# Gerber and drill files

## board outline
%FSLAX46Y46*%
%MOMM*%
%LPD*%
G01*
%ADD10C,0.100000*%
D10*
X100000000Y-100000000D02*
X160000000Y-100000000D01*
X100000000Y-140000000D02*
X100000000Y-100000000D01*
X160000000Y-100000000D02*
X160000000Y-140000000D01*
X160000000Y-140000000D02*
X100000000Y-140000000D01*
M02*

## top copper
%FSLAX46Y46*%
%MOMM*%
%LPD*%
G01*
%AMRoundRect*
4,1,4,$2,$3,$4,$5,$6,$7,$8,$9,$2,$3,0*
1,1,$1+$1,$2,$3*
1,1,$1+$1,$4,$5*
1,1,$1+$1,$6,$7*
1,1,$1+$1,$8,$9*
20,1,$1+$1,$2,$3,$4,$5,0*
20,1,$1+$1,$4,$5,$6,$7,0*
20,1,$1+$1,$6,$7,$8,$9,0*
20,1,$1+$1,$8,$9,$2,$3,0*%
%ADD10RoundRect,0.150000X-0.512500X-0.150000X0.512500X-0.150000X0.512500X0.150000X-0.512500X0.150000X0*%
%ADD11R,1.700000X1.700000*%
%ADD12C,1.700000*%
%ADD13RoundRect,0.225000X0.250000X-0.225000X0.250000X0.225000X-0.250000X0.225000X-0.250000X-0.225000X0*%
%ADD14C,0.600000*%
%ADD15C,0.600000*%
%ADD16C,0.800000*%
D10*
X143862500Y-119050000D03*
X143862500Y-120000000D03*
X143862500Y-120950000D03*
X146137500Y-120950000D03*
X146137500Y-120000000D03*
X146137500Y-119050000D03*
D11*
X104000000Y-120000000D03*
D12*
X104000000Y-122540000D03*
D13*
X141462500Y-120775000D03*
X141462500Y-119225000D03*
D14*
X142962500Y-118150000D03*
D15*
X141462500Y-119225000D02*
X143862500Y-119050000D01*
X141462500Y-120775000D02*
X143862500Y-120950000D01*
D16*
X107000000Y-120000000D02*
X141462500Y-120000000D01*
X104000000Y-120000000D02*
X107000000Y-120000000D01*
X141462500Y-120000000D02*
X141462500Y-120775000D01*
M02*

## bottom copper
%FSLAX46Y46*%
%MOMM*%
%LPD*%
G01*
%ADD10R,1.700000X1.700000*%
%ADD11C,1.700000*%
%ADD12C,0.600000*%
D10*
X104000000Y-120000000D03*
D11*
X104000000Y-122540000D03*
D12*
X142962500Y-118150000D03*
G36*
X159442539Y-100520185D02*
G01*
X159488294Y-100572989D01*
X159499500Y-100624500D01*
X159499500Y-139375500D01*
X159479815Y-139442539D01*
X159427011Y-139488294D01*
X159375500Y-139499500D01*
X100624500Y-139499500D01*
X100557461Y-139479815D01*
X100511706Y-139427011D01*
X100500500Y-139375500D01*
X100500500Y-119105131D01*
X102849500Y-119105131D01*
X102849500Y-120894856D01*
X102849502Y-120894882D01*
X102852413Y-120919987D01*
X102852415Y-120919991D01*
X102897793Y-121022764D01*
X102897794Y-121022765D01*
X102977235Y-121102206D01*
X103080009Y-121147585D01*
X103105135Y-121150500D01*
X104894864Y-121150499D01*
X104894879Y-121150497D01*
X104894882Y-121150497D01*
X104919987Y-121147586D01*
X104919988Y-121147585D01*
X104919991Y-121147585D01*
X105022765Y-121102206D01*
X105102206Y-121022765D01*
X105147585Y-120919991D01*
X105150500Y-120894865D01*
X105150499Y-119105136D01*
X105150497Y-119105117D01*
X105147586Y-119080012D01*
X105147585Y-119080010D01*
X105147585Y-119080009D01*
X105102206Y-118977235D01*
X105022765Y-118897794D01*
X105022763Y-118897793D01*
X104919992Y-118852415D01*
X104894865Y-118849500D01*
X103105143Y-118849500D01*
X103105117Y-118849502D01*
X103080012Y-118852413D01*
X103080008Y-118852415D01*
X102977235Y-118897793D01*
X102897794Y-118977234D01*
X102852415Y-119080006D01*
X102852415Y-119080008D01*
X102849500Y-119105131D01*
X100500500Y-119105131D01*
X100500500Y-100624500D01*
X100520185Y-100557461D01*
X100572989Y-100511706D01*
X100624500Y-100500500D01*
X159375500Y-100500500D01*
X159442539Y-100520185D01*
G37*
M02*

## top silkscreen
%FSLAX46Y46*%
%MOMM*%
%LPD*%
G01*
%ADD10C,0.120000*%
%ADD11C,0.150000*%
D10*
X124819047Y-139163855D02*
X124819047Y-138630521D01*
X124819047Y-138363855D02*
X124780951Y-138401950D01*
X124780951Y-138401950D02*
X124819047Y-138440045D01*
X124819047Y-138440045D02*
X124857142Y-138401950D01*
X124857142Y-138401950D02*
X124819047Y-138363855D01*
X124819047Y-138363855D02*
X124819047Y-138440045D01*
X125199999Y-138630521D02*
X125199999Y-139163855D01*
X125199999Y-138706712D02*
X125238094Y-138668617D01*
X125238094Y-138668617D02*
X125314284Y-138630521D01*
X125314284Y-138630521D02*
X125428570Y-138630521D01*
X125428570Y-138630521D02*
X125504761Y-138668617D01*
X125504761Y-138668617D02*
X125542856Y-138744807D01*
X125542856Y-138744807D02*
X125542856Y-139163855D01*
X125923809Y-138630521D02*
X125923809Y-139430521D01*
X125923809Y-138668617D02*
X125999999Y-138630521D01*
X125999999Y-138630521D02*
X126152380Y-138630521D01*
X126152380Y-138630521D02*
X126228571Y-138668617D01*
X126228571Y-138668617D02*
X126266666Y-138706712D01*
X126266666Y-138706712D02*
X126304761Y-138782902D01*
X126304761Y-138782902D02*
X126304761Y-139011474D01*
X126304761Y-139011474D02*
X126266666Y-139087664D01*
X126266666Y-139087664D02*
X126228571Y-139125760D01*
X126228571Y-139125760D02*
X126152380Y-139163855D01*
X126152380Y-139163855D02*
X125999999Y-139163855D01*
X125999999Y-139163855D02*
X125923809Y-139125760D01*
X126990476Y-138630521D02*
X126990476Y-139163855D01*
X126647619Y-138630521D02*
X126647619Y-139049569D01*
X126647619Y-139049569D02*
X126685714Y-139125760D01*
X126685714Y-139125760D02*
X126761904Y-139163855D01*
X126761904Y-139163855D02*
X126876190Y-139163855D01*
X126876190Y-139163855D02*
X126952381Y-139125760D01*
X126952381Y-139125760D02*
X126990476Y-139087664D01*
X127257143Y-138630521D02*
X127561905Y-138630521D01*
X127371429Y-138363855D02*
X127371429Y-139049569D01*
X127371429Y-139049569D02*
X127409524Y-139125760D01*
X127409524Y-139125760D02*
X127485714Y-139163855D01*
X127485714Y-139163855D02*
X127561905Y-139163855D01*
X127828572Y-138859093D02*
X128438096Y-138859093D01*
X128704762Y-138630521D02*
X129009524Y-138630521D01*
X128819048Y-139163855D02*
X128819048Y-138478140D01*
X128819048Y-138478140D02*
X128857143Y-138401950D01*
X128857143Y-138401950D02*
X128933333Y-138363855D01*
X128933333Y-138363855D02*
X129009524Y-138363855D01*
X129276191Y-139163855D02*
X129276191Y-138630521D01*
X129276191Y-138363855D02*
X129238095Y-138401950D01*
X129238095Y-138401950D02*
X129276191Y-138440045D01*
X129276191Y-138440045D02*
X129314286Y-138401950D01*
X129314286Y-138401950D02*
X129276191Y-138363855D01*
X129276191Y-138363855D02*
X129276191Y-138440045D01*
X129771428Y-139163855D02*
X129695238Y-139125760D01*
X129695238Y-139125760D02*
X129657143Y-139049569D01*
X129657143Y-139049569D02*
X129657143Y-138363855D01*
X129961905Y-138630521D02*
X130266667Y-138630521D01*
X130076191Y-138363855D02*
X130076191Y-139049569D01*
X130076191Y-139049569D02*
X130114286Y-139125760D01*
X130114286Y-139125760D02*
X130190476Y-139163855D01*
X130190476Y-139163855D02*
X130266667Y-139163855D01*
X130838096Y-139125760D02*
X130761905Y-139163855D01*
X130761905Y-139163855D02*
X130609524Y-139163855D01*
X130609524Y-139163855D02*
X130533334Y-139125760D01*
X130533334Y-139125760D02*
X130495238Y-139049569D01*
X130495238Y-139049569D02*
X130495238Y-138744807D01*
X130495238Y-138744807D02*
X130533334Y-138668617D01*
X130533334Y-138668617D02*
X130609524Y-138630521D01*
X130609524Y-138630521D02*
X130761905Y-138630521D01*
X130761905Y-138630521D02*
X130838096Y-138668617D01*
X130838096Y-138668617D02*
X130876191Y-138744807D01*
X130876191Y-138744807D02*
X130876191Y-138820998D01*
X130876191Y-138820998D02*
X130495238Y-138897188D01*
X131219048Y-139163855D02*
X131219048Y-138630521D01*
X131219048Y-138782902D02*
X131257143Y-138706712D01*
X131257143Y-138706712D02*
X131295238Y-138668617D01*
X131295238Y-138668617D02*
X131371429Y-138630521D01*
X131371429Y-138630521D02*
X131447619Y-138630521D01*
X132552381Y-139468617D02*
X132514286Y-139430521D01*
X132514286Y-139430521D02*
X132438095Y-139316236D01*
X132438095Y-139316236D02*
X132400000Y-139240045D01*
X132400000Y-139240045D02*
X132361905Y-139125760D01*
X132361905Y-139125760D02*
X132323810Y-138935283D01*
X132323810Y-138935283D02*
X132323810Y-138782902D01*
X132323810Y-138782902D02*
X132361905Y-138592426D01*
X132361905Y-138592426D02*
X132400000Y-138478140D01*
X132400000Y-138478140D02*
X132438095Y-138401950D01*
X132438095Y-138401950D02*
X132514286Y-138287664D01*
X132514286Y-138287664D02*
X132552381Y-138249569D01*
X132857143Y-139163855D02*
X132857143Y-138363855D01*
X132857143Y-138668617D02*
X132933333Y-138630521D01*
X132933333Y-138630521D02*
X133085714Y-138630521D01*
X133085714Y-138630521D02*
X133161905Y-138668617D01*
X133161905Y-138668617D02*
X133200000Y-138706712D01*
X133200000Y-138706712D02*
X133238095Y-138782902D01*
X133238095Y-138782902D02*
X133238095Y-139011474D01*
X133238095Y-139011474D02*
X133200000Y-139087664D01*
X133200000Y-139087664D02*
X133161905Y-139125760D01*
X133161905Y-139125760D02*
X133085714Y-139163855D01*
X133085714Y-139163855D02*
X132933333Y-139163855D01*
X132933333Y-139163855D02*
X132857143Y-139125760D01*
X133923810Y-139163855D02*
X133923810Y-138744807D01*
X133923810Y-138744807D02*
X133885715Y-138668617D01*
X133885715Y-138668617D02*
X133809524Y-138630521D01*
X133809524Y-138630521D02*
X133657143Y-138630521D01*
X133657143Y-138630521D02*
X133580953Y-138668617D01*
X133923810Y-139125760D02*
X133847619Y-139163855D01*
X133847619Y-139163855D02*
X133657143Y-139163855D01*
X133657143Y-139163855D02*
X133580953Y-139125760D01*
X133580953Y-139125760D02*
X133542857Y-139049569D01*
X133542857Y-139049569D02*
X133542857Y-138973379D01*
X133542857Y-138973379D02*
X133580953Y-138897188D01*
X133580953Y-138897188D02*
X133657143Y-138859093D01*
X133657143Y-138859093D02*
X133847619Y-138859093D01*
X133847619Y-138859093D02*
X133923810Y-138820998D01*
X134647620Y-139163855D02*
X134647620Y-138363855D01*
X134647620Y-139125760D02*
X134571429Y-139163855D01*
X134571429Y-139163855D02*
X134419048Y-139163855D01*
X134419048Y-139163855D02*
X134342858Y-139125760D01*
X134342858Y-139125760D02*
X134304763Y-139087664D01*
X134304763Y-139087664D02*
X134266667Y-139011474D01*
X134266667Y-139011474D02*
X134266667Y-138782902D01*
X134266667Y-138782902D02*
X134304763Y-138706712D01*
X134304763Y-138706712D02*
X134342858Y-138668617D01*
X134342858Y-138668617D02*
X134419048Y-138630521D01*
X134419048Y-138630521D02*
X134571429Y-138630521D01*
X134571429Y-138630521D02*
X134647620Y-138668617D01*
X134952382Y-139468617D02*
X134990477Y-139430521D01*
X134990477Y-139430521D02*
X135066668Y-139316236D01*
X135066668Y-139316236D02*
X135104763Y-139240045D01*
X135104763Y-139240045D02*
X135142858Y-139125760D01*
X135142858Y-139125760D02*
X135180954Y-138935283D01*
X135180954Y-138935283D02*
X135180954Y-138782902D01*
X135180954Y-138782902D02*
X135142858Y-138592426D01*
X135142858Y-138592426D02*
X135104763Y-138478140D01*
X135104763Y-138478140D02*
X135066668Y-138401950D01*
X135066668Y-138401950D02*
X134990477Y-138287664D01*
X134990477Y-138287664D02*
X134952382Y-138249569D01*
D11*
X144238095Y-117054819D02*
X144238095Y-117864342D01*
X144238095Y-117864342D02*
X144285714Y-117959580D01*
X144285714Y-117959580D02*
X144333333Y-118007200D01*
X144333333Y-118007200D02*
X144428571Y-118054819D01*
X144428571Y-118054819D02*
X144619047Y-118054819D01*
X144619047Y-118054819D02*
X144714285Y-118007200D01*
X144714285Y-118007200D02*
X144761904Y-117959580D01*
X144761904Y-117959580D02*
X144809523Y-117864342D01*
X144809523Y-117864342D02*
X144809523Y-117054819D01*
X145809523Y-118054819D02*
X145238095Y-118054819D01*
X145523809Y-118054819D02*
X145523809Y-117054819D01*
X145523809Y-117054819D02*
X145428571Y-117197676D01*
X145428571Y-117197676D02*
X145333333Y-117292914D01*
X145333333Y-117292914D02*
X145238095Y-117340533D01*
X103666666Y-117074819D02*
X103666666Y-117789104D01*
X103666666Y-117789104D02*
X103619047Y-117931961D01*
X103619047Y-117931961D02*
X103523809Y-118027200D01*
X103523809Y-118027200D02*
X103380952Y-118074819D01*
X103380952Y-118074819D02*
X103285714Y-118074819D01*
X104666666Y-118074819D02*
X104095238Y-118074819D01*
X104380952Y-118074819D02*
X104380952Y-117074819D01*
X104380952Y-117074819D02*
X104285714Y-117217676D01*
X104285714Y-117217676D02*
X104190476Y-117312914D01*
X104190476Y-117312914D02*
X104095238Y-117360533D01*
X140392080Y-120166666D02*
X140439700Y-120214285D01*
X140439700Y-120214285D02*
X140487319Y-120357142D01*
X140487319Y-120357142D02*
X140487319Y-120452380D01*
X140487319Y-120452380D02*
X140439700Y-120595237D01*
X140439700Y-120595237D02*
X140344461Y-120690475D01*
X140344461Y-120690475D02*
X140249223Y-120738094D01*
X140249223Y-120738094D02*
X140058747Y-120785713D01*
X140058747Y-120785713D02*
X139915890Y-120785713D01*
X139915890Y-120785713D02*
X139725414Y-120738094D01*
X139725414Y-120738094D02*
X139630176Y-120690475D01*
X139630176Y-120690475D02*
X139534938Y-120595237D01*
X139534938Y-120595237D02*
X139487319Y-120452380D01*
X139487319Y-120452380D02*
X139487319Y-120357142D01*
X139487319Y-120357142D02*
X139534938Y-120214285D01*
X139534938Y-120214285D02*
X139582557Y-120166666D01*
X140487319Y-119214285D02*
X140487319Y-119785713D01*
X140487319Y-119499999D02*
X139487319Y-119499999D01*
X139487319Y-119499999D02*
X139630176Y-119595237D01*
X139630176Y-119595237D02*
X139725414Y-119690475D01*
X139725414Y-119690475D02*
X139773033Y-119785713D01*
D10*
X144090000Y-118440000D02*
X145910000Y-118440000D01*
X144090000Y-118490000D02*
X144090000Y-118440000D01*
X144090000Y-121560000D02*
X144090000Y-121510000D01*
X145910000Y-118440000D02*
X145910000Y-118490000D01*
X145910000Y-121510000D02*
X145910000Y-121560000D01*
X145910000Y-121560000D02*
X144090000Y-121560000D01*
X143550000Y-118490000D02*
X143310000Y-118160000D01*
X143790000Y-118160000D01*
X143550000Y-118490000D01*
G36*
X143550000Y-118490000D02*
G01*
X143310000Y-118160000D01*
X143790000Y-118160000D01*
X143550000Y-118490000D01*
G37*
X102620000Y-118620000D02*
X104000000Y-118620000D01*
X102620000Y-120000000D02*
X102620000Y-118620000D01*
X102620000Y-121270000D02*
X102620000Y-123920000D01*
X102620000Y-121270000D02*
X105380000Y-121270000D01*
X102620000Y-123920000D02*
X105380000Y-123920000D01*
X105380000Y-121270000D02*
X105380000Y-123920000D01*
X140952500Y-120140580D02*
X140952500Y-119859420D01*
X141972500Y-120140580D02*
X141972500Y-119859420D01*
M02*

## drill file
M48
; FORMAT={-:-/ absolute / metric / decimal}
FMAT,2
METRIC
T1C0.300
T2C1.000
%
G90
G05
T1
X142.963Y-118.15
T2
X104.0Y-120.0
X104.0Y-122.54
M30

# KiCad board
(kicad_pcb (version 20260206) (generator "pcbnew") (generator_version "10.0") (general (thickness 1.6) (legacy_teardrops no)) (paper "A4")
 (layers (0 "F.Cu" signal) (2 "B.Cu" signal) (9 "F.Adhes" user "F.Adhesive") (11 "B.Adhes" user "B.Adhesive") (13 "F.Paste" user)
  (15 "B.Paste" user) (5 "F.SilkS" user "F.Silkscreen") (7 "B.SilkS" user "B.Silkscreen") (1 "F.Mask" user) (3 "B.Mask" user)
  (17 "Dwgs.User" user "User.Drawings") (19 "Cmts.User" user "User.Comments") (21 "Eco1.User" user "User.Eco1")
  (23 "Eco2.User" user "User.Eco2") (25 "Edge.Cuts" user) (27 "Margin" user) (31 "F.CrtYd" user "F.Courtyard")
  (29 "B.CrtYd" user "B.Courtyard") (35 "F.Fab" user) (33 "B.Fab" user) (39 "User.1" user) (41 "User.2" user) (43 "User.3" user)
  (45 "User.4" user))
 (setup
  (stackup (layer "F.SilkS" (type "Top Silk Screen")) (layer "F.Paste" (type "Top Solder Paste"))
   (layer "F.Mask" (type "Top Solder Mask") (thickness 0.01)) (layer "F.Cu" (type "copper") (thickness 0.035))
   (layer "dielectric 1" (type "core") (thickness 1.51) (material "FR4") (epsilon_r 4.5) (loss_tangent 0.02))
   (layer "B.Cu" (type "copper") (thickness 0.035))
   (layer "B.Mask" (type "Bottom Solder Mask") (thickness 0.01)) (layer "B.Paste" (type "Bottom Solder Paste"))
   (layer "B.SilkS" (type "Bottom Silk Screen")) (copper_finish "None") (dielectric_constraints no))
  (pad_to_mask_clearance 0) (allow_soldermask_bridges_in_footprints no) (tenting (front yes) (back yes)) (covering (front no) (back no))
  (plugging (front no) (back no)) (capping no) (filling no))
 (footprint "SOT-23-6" (layer "F.Cu") (at 145 120)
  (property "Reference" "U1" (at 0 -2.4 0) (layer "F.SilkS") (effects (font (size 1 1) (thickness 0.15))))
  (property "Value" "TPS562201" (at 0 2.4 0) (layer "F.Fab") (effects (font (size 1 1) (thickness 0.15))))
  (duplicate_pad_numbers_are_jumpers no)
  (fp_line (start -0.91 -1.56) (end 0.91 -1.56) (stroke (width 0.12) (type solid)) (layer "F.SilkS"))
  (fp_line (start -0.91 -1.51) (end -0.91 -1.56) (stroke (width 0.12) (type solid)) (layer "F.SilkS"))
  (fp_line (start -0.91 1.56) (end -0.91 1.51) (stroke (width 0.12) (type solid)) (layer "F.SilkS"))
  (fp_line (start 0.91 -1.56) (end 0.91 -1.51) (stroke (width 0.12) (type solid)) (layer "F.SilkS"))
  (fp_line (start 0.91 1.51) (end 0.91 1.56) (stroke (width 0.12) (type solid)) (layer "F.SilkS"))
  (fp_line (start 0.91 1.56) (end -0.91 1.56) (stroke (width 0.12) (type solid)) (layer "F.SilkS"))
  (fp_poly (pts (xy -1.45 -1.51) (xy -1.69 -1.84) (xy -1.21 -1.84)) (stroke (width 0.12) (type solid)) (fill yes) (layer "F.SilkS"))
  (pad "1" smd roundrect (at -1.1375 -0.95) (size 1.325 0.6) (layers "F.Cu" "F.Mask" "F.Paste") (roundrect_rratio 0.25) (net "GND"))
  (pad "2" smd roundrect (at -1.1375 0) (size 1.325 0.6) (layers "F.Cu" "F.Mask" "F.Paste") (roundrect_rratio 0.25) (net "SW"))
  (pad "3" smd roundrect (at -1.1375 0.95) (size 1.325 0.6) (layers "F.Cu" "F.Mask" "F.Paste") (roundrect_rratio 0.25) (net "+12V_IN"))
  (pad "4" smd roundrect (at 1.1375 0.95) (size 1.325 0.6) (layers "F.Cu" "F.Mask" "F.Paste") (roundrect_rratio 0.25) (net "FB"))
  (pad "5" smd roundrect (at 1.1375 0) (size 1.325 0.6) (layers "F.Cu" "F.Mask" "F.Paste") (roundrect_rratio 0.25) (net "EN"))
  (pad "6" smd roundrect (at 1.1375 -0.95) (size 1.325 0.6) (layers "F.Cu" "F.Mask" "F.Paste") (roundrect_rratio 0.25) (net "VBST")))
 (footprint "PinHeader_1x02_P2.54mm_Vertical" (layer "F.Cu") (at 104 120)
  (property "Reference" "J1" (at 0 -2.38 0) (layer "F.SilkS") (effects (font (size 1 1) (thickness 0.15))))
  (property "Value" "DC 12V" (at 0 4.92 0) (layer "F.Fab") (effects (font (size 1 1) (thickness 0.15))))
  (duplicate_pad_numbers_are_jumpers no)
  (fp_line (start -1.38 -1.38) (end 0 -1.38) (stroke (width 0.12) (type solid)) (layer "F.SilkS"))
  (fp_line (start -1.38 0) (end -1.38 -1.38) (stroke (width 0.12) (type solid)) (layer "F.SilkS"))
  (fp_line (start -1.38 1.27) (end -1.38 3.92) (stroke (width 0.12) (type solid)) (layer "F.SilkS"))
  (fp_line (start -1.38 1.27) (end 1.38 1.27) (stroke (width 0.12) (type solid)) (layer "F.SilkS"))
  (fp_line (start -1.38 3.92) (end 1.38 3.92) (stroke (width 0.12) (type solid)) (layer "F.SilkS"))
  (fp_line (start 1.38 1.27) (end 1.38 3.92) (stroke (width 0.12) (type solid)) (layer "F.SilkS"))
  (pad "1" thru_hole rect (at 0 0) (size 1.7 1.7) (drill 1) (layers "*.Cu" "*.Mask") (remove_unused_layers no) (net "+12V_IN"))
  (pad "2" thru_hole circle (at 0 2.54) (size 1.7 1.7) (drill 1) (layers "*.Cu" "*.Mask") (remove_unused_layers no) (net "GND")))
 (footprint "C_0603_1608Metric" (layer "F.Cu") (at 141.4625 120 90)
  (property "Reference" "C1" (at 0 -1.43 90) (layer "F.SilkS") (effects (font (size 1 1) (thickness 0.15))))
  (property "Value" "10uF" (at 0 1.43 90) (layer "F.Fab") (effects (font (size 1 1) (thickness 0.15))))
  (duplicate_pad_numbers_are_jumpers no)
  (fp_line (start -0.14058 -0.51) (end 0.14058 -0.51) (stroke (width 0.12) (type solid)) (layer "F.SilkS"))
  (fp_line (start -0.14058 0.51) (end 0.14058 0.51) (stroke (width 0.12) (type solid)) (layer "F.SilkS"))
  (pad "1" smd roundrect (at -0.775 0 90) (size 0.9 0.95) (layers "F.Cu" "F.Mask" "F.Paste") (roundrect_rratio 0.25) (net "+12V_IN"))
  (pad "2" smd roundrect (at 0.775 0 90) (size 0.9 0.95) (layers "F.Cu" "F.Mask" "F.Paste") (roundrect_rratio 0.25) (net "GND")))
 (gr_line (start 100 100) (end 160 100) (stroke (width 0.1) (type default)) (layer "Edge.Cuts"))
 (gr_line (start 100 140) (end 100 100) (stroke (width 0.1) (type default)) (layer "Edge.Cuts"))
 (gr_line (start 160 100) (end 160 140) (stroke (width 0.1) (type default)) (layer "Edge.Cuts"))
 (gr_line (start 160 140) (end 100 140) (stroke (width 0.1) (type default)) (layer "Edge.Cuts"))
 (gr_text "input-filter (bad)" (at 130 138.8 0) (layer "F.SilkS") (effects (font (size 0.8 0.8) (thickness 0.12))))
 (segment (start 141.4625 119.225) (end 143.8625 119.05) (width 0.6) (layer "F.Cu") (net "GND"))
 (via (at 142.9625 118.15) (size 0.6) (drill 0.3) (layers "F.Cu" "B.Cu") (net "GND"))
 (segment (start 141.4625 120.775) (end 143.8625 120.95) (width 0.6) (layer "F.Cu") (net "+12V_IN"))
 (segment (start 107 120) (end 141.4625 120) (width 0.8) (layer "F.Cu") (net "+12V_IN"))
 (segment (start 104 120) (end 107 120) (width 0.8) (layer "F.Cu") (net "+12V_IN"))
 (segment (start 141.4625 120) (end 141.4625 120.775) (width 0.8) (layer "F.Cu") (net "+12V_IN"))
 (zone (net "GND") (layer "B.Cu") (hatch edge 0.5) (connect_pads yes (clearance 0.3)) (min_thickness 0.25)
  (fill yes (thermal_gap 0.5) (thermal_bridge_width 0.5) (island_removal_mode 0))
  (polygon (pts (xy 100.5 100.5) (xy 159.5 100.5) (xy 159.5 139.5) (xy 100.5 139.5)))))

